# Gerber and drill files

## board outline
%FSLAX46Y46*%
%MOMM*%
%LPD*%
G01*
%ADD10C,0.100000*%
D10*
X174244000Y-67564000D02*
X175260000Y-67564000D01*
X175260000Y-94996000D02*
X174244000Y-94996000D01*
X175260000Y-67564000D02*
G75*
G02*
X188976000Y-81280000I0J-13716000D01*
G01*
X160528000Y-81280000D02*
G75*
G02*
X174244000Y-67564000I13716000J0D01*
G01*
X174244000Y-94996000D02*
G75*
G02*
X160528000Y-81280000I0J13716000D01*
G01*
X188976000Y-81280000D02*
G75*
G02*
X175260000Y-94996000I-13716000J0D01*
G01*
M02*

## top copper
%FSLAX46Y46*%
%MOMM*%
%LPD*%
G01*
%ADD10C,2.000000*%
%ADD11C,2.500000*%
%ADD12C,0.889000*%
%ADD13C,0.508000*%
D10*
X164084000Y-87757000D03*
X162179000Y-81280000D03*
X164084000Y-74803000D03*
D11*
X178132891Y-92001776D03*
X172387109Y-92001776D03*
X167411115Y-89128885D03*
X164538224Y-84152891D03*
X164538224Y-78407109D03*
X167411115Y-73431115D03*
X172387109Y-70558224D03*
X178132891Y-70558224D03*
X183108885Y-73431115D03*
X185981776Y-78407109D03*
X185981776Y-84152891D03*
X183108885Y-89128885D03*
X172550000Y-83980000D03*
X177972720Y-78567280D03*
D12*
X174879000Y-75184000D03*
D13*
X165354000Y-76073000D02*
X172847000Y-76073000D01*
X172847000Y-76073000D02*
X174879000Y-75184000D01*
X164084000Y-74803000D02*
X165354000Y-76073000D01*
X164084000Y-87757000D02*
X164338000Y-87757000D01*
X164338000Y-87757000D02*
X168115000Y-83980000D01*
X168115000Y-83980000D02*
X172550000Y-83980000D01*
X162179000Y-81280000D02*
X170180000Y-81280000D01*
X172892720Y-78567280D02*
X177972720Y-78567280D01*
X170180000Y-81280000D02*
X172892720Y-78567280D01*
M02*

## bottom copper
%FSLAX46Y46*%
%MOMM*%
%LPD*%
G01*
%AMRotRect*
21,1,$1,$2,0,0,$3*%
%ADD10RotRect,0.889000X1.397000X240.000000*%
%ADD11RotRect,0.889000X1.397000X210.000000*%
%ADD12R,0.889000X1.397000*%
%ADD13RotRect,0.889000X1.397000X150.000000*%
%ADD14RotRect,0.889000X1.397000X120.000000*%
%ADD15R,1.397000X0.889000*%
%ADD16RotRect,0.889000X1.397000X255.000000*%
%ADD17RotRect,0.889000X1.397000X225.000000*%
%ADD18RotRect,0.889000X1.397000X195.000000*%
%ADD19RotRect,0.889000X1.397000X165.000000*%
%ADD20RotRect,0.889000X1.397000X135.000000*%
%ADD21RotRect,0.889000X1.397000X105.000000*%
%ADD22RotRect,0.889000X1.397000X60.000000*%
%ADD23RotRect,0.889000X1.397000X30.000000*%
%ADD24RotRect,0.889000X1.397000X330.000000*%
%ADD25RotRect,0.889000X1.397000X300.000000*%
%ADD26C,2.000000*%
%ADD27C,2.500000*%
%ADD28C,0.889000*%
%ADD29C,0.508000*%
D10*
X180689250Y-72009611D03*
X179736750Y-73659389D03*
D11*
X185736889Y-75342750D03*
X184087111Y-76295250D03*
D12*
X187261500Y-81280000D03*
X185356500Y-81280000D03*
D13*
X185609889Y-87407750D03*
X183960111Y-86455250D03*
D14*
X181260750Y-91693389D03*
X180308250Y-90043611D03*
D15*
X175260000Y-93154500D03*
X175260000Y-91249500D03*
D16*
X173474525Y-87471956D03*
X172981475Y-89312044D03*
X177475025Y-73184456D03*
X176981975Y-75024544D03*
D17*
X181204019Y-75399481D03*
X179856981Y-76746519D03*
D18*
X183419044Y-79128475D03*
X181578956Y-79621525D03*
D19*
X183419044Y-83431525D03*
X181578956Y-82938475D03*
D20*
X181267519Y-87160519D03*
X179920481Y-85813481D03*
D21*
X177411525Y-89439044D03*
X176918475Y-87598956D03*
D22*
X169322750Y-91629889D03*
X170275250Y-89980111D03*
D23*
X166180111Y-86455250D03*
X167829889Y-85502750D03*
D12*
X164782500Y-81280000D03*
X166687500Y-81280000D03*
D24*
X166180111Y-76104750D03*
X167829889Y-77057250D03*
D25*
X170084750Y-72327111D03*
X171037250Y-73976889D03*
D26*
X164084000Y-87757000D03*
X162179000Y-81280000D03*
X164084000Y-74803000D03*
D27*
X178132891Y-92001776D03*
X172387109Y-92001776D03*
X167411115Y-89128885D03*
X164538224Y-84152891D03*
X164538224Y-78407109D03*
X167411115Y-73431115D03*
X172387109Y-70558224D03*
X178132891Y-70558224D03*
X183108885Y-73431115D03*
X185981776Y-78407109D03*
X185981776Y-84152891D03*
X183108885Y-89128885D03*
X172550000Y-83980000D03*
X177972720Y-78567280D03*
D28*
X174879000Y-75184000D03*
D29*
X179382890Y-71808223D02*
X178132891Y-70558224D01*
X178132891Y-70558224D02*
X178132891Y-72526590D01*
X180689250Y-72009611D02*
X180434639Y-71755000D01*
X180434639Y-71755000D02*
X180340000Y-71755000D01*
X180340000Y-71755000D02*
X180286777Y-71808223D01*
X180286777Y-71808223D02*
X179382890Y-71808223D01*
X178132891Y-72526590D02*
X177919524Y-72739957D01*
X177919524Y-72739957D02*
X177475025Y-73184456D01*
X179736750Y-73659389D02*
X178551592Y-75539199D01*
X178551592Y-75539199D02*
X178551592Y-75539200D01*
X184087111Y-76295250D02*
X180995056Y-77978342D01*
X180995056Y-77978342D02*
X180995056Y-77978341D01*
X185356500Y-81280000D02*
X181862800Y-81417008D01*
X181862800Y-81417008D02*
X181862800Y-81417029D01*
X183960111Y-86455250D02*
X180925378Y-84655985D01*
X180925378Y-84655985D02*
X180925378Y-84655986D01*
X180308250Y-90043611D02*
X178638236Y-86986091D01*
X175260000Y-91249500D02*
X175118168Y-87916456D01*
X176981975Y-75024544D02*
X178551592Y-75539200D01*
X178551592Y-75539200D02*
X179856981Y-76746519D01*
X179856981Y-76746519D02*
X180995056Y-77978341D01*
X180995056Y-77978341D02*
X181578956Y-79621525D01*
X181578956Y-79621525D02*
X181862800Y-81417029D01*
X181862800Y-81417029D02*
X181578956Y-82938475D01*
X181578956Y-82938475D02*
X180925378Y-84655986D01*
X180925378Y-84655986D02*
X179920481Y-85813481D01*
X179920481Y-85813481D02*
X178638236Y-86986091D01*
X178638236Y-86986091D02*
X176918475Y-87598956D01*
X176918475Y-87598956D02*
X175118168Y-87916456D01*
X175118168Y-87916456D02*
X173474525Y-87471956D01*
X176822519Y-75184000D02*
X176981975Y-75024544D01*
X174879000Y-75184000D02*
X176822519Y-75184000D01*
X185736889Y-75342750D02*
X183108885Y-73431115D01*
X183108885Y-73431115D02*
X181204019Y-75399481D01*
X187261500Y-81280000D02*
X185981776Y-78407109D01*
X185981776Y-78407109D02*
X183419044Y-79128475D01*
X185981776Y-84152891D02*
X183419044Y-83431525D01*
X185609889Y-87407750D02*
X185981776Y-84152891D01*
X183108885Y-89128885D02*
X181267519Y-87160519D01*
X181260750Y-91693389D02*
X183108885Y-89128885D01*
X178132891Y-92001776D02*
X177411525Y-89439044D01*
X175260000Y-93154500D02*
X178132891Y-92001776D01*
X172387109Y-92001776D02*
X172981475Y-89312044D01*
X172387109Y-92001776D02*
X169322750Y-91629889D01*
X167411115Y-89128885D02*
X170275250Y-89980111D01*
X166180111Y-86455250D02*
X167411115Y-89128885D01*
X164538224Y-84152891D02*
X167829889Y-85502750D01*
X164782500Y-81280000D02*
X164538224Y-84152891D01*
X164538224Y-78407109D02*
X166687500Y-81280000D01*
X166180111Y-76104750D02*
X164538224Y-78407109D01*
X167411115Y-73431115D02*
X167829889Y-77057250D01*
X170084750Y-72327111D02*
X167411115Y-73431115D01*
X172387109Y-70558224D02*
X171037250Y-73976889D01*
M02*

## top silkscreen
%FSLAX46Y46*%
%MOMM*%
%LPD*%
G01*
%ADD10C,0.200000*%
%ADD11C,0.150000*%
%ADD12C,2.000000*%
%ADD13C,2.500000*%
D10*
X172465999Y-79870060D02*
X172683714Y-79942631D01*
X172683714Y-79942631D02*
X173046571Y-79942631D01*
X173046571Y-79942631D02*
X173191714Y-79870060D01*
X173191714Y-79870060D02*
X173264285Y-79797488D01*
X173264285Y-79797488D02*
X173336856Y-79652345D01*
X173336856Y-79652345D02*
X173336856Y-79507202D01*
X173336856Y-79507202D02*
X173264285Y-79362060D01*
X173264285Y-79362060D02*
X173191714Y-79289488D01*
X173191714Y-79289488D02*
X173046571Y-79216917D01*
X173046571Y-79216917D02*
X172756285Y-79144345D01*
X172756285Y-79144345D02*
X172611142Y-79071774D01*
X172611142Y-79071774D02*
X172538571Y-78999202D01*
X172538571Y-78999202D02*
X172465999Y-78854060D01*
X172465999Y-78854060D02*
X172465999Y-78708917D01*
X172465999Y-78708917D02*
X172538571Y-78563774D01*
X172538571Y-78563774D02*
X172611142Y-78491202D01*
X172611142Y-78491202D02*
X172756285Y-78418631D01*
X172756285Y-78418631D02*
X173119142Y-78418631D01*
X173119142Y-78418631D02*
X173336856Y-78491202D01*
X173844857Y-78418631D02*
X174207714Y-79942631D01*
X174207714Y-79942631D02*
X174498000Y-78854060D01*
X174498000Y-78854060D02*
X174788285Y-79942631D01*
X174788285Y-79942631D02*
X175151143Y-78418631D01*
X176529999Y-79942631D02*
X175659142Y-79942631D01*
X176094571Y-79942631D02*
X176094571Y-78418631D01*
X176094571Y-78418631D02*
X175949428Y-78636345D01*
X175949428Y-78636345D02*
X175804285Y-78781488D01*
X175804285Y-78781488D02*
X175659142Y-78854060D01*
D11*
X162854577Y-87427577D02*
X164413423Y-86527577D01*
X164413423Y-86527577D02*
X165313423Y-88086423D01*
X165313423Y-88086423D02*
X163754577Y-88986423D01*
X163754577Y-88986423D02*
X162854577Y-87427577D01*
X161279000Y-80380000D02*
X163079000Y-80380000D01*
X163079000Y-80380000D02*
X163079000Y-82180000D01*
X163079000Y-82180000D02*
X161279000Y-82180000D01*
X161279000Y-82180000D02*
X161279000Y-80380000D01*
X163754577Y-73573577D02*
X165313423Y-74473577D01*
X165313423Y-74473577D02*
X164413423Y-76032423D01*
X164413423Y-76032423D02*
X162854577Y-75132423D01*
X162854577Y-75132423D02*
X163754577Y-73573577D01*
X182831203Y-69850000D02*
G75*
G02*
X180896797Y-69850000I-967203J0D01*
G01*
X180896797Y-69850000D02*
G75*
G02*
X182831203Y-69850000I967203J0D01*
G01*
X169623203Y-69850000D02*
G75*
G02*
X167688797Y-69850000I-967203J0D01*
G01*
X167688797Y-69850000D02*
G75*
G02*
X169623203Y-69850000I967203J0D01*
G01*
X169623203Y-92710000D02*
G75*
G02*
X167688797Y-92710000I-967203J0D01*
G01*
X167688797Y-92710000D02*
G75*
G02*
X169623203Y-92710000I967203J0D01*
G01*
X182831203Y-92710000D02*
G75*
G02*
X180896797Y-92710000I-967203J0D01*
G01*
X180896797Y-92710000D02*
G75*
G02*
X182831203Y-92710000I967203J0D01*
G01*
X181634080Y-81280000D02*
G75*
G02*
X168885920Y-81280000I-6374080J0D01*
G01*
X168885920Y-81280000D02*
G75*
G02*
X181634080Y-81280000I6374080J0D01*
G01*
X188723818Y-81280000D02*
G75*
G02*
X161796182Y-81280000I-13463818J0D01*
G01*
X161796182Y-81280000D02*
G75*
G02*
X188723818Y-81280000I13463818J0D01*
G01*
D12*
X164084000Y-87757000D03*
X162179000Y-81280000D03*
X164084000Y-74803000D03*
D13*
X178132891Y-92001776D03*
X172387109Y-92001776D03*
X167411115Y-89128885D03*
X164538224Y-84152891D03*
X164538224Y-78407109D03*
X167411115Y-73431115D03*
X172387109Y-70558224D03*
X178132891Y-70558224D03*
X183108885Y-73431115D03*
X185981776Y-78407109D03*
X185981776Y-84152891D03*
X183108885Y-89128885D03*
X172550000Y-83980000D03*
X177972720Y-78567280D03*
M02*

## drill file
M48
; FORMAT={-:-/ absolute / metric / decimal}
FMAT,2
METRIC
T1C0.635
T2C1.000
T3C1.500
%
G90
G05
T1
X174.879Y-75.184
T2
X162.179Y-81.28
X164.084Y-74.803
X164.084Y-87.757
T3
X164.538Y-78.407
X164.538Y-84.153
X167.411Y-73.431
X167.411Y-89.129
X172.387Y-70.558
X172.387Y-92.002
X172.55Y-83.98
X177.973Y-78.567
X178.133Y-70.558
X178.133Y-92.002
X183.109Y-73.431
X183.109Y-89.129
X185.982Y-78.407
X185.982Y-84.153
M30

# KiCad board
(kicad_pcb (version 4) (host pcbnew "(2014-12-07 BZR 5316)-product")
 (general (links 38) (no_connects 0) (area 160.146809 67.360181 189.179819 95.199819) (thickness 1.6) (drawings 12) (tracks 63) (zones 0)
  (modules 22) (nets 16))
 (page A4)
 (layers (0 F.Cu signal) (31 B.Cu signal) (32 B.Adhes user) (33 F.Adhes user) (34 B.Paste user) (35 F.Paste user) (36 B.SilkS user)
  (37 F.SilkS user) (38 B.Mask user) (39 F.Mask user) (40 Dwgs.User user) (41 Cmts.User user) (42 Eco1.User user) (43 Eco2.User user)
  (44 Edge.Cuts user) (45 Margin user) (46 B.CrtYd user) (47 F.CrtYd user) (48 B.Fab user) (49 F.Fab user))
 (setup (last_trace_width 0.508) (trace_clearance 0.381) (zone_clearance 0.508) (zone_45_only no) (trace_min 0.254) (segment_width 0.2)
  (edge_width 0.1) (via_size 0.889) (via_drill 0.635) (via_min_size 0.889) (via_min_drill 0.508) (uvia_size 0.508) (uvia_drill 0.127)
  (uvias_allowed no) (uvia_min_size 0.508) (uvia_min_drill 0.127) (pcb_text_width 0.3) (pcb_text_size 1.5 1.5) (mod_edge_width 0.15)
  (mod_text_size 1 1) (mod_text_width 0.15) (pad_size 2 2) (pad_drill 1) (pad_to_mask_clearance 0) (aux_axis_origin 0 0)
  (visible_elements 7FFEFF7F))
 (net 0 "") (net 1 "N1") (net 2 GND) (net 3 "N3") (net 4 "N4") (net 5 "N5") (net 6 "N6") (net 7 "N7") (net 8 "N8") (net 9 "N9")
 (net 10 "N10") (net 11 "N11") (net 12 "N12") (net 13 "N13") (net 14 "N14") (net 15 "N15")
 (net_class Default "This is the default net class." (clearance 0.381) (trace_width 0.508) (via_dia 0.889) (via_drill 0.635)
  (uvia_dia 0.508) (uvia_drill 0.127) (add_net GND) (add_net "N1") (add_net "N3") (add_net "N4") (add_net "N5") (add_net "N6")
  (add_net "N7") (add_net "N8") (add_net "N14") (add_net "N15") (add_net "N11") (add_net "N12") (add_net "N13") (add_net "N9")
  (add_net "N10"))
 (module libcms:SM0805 (layer B.Cu) (at 180.213 72.8345 240)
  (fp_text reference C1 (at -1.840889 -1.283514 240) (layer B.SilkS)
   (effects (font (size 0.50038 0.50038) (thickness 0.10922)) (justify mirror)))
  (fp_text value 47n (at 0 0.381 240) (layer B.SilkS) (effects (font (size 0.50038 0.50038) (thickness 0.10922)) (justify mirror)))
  (pad 1 smd rect (at -0.9525 0 240) (size 0.889 1.397) (layers B.Cu B.Paste B.Mask) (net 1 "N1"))
  (pad 2 smd rect (at 0.9525 0 240) (size 0.889 1.397) (layers B.Cu B.Paste B.Mask) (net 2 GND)))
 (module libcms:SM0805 (layer B.Cu) (at 184.912 75.819 210)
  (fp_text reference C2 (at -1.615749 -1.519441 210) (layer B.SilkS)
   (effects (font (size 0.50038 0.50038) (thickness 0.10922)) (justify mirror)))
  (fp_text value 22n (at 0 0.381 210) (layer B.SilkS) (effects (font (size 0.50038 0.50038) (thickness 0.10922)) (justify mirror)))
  (pad 1 smd rect (at -0.9525 0 210) (size 0.889 1.397) (layers B.Cu B.Paste B.Mask) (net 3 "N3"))
  (pad 2 smd rect (at 0.9525 0 210) (size 0.889 1.397) (layers B.Cu B.Paste B.Mask) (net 2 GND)))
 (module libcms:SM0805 (layer B.Cu) (at 186.309 81.28 180)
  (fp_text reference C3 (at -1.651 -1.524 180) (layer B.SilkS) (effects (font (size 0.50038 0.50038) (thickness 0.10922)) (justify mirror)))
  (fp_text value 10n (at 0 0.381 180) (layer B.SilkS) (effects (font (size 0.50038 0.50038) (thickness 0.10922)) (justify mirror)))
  (pad 1 smd rect (at -0.9525 0 180) (size 0.889 1.397) (layers B.Cu B.Paste B.Mask) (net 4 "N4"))
  (pad 2 smd rect (at 0.9525 0 180) (size 0.889 1.397) (layers B.Cu B.Paste B.Mask) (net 2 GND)))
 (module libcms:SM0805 (layer B.Cu) (at 184.785 86.9315 150)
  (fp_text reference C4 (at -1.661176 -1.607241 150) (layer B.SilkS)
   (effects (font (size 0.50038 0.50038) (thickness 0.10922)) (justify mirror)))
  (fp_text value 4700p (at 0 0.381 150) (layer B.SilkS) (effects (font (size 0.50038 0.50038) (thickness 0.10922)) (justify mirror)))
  (pad 1 smd rect (at -0.9525 0 150) (size 0.889 1.397) (layers B.Cu B.Paste B.Mask) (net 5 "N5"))
  (pad 2 smd rect (at 0.9525 0 150) (size 0.889 1.397) (layers B.Cu B.Paste B.Mask) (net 2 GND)))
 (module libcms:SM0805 (layer B.Cu) (at 180.7845 90.8685 120)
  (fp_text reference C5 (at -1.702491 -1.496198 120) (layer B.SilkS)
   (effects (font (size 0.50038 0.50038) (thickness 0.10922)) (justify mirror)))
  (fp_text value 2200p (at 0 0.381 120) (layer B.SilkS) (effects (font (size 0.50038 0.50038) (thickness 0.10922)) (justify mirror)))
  (pad 1 smd rect (at -0.9525 0 120) (size 0.889 1.397) (layers B.Cu B.Paste B.Mask) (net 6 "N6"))
  (pad 2 smd rect (at 0.9525 0 120) (size 0.889 1.397) (layers B.Cu B.Paste B.Mask) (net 2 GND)))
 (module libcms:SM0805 (layer B.Cu) (at 175.26 92.202 90)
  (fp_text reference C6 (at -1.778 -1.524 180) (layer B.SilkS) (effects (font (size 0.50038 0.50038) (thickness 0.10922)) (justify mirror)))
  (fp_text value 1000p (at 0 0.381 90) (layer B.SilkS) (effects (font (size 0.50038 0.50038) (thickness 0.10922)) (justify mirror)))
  (pad 1 smd rect (at -0.9525 0 90) (size 0.889 1.397) (layers B.Cu B.Paste B.Mask) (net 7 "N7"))
  (pad 2 smd rect (at 0.9525 0 90) (size 0.889 1.397) (layers B.Cu B.Paste B.Mask) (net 2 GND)))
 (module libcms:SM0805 (layer B.Cu) (at 173.228 88.392 255)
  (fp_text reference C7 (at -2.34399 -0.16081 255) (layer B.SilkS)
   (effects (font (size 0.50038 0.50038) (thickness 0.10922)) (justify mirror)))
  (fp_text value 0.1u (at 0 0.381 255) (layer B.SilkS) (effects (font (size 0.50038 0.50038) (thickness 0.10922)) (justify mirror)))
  (pad 1 smd rect (at -0.9525 0 255) (size 0.889 1.397) (layers B.Cu B.Paste B.Mask) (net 2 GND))
  (pad 2 smd rect (at 0.9525 0 255) (size 0.889 1.397) (layers B.Cu B.Paste B.Mask) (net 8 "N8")))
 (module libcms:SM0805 (layer B.Cu) (at 177.2285 74.1045 255)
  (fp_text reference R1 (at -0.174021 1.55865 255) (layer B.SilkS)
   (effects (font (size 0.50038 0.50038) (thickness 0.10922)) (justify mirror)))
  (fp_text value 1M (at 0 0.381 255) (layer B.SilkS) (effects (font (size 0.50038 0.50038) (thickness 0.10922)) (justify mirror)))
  (pad 1 smd rect (at -0.9525 0 255) (size 0.889 1.397) (layers B.Cu B.Paste B.Mask) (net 1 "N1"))
  (pad 2 smd rect (at 0.9525 0 255) (size 0.889 1.397) (layers B.Cu B.Paste B.Mask) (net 2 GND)))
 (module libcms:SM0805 (layer B.Cu) (at 180.5305 76.073 225)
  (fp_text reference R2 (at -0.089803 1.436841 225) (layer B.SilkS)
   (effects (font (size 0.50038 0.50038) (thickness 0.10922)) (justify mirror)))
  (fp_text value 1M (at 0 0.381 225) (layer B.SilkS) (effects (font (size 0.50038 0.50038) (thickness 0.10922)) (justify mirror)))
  (pad 1 smd rect (at -0.9525 0 225) (size 0.889 1.397) (layers B.Cu B.Paste B.Mask) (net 3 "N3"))
  (pad 2 smd rect (at 0.9525 0 225) (size 0.889 1.397) (layers B.Cu B.Paste B.Mask) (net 2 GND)))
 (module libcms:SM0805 (layer B.Cu) (at 182.499 79.375 195)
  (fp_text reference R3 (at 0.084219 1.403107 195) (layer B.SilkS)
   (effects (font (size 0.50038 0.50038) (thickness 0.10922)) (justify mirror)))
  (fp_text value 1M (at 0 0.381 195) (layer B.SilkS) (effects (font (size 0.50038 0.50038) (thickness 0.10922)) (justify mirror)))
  (pad 1 smd rect (at -0.9525 0 195) (size 0.889 1.397) (layers B.Cu B.Paste B.Mask) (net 4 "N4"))
  (pad 2 smd rect (at 0.9525 0 195) (size 0.889 1.397) (layers B.Cu B.Paste B.Mask) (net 2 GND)))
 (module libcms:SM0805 (layer B.Cu) (at 182.499 83.185 165)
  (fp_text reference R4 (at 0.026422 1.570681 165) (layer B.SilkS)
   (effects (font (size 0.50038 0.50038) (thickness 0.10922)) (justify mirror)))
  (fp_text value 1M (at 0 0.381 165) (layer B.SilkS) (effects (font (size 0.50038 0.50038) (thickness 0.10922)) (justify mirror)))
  (pad 1 smd rect (at -0.9525 0 165) (size 0.889 1.397) (layers B.Cu B.Paste B.Mask) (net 5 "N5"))
  (pad 2 smd rect (at 0.9525 0 165) (size 0.889 1.397) (layers B.Cu B.Paste B.Mask) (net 2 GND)))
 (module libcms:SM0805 (layer B.Cu) (at 180.594 86.487 135)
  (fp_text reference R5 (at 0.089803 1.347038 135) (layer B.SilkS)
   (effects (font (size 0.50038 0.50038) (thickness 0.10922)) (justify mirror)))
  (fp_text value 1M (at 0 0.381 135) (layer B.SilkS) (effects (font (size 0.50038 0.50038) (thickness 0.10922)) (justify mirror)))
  (pad 1 smd rect (at -0.9525 0 135) (size 0.889 1.397) (layers B.Cu B.Paste B.Mask) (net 6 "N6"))
  (pad 2 smd rect (at 0.9525 0 135) (size 0.889 1.397) (layers B.Cu B.Paste B.Mask) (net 2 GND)))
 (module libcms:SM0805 (layer B.Cu) (at 177.165 88.519 105)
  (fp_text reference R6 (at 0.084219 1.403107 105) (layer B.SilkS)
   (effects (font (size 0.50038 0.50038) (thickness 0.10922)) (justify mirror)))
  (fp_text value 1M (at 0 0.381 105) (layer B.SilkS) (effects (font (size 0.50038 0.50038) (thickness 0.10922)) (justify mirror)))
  (pad 1 smd rect (at -0.9525 0 105) (size 0.889 1.397) (layers B.Cu B.Paste B.Mask) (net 7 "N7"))
  (pad 2 smd rect (at 0.9525 0 105) (size 0.889 1.397) (layers B.Cu B.Paste B.Mask) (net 2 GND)))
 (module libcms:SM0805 (layer B.Cu) (at 169.799 90.805 60)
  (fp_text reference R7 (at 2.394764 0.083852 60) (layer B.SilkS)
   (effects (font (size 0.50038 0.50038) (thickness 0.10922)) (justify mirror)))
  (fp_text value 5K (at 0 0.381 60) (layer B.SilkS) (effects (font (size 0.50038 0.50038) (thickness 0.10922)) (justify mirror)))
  (pad 1 smd rect (at -0.9525 0 60) (size 0.889 1.397) (layers B.Cu B.Paste B.Mask) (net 8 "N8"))
  (pad 2 smd rect (at 0.9525 0 60) (size 0.889 1.397) (layers B.Cu B.Paste B.Mask) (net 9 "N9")))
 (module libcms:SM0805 (layer B.Cu) (at 167.005 85.979 30)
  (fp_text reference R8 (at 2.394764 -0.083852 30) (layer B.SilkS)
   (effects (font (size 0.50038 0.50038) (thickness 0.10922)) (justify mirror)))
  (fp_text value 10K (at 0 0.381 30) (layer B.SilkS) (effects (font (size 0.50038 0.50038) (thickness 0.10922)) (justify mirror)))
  (pad 1 smd rect (at -0.9525 0 30) (size 0.889 1.397) (layers B.Cu B.Paste B.Mask) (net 9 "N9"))
  (pad 2 smd rect (at 0.9525 0 30) (size 0.889 1.397) (layers B.Cu B.Paste B.Mask) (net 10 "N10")))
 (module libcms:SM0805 (layer B.Cu) (at 165.735 81.28)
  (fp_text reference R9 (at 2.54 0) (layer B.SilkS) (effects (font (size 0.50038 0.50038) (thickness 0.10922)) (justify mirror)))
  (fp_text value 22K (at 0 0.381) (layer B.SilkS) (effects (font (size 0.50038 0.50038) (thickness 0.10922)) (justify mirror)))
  (pad 1 smd rect (at -0.9525 0) (size 0.889 1.397) (layers B.Cu B.Paste B.Mask) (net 10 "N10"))
  (pad 2 smd rect (at 0.9525 0) (size 0.889 1.397) (layers B.Cu B.Paste B.Mask) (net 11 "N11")))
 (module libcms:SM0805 (layer B.Cu) (at 167.005 76.581 330)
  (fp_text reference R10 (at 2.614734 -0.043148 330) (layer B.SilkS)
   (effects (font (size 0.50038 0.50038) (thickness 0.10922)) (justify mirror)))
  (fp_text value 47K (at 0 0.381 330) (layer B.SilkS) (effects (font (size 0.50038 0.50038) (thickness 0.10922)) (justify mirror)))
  (pad 1 smd rect (at -0.9525 0 330) (size 0.889 1.397) (layers B.Cu B.Paste B.Mask) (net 11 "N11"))
  (pad 2 smd rect (at 0.9525 0 330) (size 0.889 1.397) (layers B.Cu B.Paste B.Mask) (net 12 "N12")))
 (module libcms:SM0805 (layer B.Cu) (at 170.561 73.152 300)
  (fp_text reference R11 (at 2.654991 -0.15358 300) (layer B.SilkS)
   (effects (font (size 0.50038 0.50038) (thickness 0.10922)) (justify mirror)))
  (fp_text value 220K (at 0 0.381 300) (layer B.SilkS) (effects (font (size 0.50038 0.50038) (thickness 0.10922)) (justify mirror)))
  (pad 1 smd rect (at -0.9525 0 300) (size 0.889 1.397) (layers B.Cu B.Paste B.Mask) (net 12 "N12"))
  (pad 2 smd rect (at 0.9525 0 300) (size 0.889 1.397) (layers B.Cu B.Paste B.Mask) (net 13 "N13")))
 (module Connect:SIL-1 (layer F.Cu) (at 164.084 87.757 30)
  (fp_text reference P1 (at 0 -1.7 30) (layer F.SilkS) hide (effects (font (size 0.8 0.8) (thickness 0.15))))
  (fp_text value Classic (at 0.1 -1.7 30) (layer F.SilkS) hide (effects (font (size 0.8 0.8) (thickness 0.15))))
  (fp_line (start -0.9 -0.9) (end 0.9 -0.9) (layer F.SilkS) (width 0.15))
  (fp_line (start 0.9 -0.9) (end 0.9 0.9) (layer F.SilkS) (width 0.15))
  (fp_line (start 0.9 0.9) (end -0.9 0.9) (layer F.SilkS) (width 0.15))
  (fp_line (start -0.9 0.9) (end -0.9 -0.9) (layer F.SilkS) (width 0.15))
  (pad 1 thru_hole circle (at 0 0 30) (size 2 2) (drill 1) (layers *.Cu *.Mask F.SilkS) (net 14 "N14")))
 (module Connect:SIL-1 (layer F.Cu) (at 162.179 81.28)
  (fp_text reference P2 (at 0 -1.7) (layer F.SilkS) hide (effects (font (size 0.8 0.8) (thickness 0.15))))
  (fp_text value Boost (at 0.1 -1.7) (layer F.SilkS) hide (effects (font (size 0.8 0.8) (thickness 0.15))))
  (fp_line (start -0.9 -0.9) (end 0.9 -0.9) (layer F.SilkS) (width 0.15))
  (fp_line (start 0.9 -0.9) (end 0.9 0.9) (layer F.SilkS) (width 0.15))
  (fp_line (start 0.9 0.9) (end -0.9 0.9) (layer F.SilkS) (width 0.15))
  (fp_line (start -0.9 0.9) (end -0.9 -0.9) (layer F.SilkS) (width 0.15))
  (pad 1 thru_hole circle (at 0 0) (size 2 2) (drill 1) (layers *.Cu *.Mask F.SilkS) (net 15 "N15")))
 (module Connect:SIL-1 (layer F.Cu) (at 164.084 74.803 330)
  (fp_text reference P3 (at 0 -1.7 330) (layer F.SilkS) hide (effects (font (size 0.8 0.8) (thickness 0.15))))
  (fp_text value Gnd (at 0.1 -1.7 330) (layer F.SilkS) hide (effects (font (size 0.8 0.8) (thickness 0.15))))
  (fp_line (start -0.9 -0.9) (end 0.9 -0.9) (layer F.SilkS) (width 0.15))
  (fp_line (start 0.9 -0.9) (end 0.9 0.9) (layer F.SilkS) (width 0.15))
  (fp_line (start 0.9 0.9) (end -0.9 0.9) (layer F.SilkS) (width 0.15))
  (fp_line (start -0.9 0.9) (end -0.9 -0.9) (layer F.SilkS) (width 0.15))
  (pad 1 thru_hole circle (at 0 0 330) (size 2 2) (drill 1) (layers *.Cu *.Mask F.SilkS) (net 2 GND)))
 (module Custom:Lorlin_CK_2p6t (layer F.Cu) (at 175.26 81.28)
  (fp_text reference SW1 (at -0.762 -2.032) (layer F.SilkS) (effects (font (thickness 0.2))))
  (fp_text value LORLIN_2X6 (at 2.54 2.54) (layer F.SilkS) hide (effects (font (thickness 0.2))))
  (fp_circle (center 6.604 -11.43) (end 7.493 -11.049) (layer F.SilkS) (width 0.15))
  (fp_circle (center -6.604 -11.43) (end -5.715 -11.049) (layer F.SilkS) (width 0.15))
  (fp_circle (center -6.604 11.43) (end -5.715 11.811) (layer F.SilkS) (width 0.15))
  (fp_circle (center 6.604 11.43) (end 7.493 11.811) (layer F.SilkS) (width 0.15))
  (fp_circle (center 0 0) (end 5.08 3.85) (layer F.SilkS) (width 0.15))
  (fp_circle (center 0 0) (end 11.1 7.62) (layer F.SilkS) (width 0.15))
  (pad 12 thru_hole circle (at 2.872891 10.721776) (size 2.5 2.5) (drill 1.5) (layers *.Cu *.Mask F.SilkS) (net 7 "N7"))
  (pad 1 thru_hole circle (at -2.872891 10.721776) (size 2.5 2.5) (drill 1.5) (layers *.Cu *.Mask F.SilkS) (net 8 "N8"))
  (pad 2 thru_hole circle (at -7.848885 7.848885) (size 2.5 2.5) (drill 1.5) (layers *.Cu *.Mask F.SilkS) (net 9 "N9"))
  (pad 3 thru_hole circle (at -10.721776 2.872891) (size 2.5 2.5) (drill 1.5) (layers *.Cu *.Mask F.SilkS) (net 10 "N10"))
  (pad 4 thru_hole circle (at -10.721776 -2.872891) (size 2.5 2.5) (drill 1.5) (layers *.Cu *.Mask F.SilkS) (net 11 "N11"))
  (pad 5 thru_hole circle (at -7.848885 -7.848885) (size 2.5 2.5) (drill 1.5) (layers *.Cu *.Mask F.SilkS) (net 12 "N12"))
  (pad 6 thru_hole circle (at -2.872891 -10.721776) (size 2.5 2.5) (drill 1.5) (layers *.Cu *.Mask F.SilkS) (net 13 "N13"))
  (pad 7 thru_hole circle (at 2.872891 -10.721776) (size 2.5 2.5) (drill 1.5) (layers *.Cu *.Mask F.SilkS) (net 1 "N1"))
  (pad 8 thru_hole circle (at 7.848885 -7.848885) (size 2.5 2.5) (drill 1.5) (layers *.Cu *.Mask F.SilkS) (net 3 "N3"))
  (pad 9 thru_hole circle (at 10.721776 -2.872891) (size 2.5 2.5) (drill 1.5) (layers *.Cu *.Mask F.SilkS) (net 4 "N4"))
  (pad 10 thru_hole circle (at 10.721776 2.872891) (size 2.5 2.5) (drill 1.5) (layers *.Cu *.Mask F.SilkS) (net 5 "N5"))
  (pad 11 thru_hole circle (at 7.848885 7.848885) (size 2.5 2.5) (drill 1.5) (layers *.Cu *.Mask F.SilkS) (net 6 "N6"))
  (pad A thru_hole circle (at -2.71 2.7) (size 2.5 2.5) (drill 1.5) (layers *.Cu *.Mask F.SilkS) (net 14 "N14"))
  (pad B thru_hole circle (at 2.71272 -2.71272) (size 2.5 2.5) (drill 1.5) (layers *.Cu *.Mask F.SilkS) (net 15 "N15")))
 (gr_line (start 174.244 67.564) (end 175.26 67.564) (angle 90) (layer Edge.Cuts) (width 0.1))
 (gr_line (start 175.26 94.996) (end 174.244 94.996) (angle 90) (layer Edge.Cuts) (width 0.1))
 (gr_arc (start 175.26 81.28) (end 175.26 67.564) (angle 90) (layer Edge.Cuts) (width 0.1))
 (gr_arc (start 174.244 81.28) (end 160.528 81.28) (angle 90) (layer Edge.Cuts) (width 0.1))
 (gr_arc (start 174.244 81.28) (end 174.244 94.996) (angle 90) (layer Edge.Cuts) (width 0.1))
 (gr_arc (start 175.26 81.28) (end 188.976 81.28) (angle 90) (layer Edge.Cuts) (width 0.1))
 (segment (start 179.38289 71.808223) (end 178.132891 70.558224) (width 0.508) (layer B.Cu) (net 1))
 (segment (start 178.132891 70.558224) (end 178.132891 72.52659) (width 0.508) (layer B.Cu) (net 1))
 (segment (start 180.68925 72.009611) (end 180.434639 71.755) (width 0.508) (layer B.Cu) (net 1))
 (segment (start 180.434639 71.755) (end 180.34 71.755) (width 0.508) (layer B.Cu) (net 1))
 (segment (start 180.34 71.755) (end 180.286777 71.808223) (width 0.508) (layer B.Cu) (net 1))
 (segment (start 180.286777 71.808223) (end 179.38289 71.808223) (width 0.508) (layer B.Cu) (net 1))
 (segment (start 178.132891 72.52659) (end 177.919524 72.739957) (width 0.508) (layer B.Cu) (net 1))
 (segment (start 177.919524 72.739957) (end 177.475025 73.184456) (width 0.508) (layer B.Cu) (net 1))
 (segment (start 179.73675 73.659389) (end 178.551592 75.539199) (width 0.508) (layer B.Cu) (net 2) (status 10))
 (segment (start 178.551592 75.539199) (end 178.551592 75.5392) (width 0.508) (layer B.Cu) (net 2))
 (segment (start 184.087111 76.29525) (end 180.995056 77.978342) (width 0.508) (layer B.Cu) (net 2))
 (segment (start 180.995056 77.978342) (end 180.995056 77.978341) (width 0.508) (layer B.Cu) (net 2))
 (segment (start 185.3565 81.28) (end 181.8628 81.417008) (width 0.508) (layer B.Cu) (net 2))
 (segment (start 181.8628 81.417008) (end 181.8628 81.417029) (width 0.508) (layer B.Cu) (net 2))
 (segment (start 183.960111 86.45525) (end 180.925378 84.655985) (width 0.508) (layer B.Cu) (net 2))
 (segment (start 180.925378 84.655985) (end 180.925378 84.655986) (width 0.508) (layer B.Cu) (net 2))
 (segment (start 180.30825 90.043611) (end 178.638236 86.986091) (width 0.508) (layer B.Cu) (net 2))
 (segment (start 175.26 91.2495) (end 175.118168 87.916456) (width 0.508) (layer B.Cu) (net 2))
 (segment (start 176.981975 75.024544) (end 178.551592 75.5392) (width 0.508) (layer B.Cu) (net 2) (status 10))
 (segment (start 178.551592 75.5392) (end 179.856981 76.746519) (width 0.508) (layer B.Cu) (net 2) (status 20))
 (segment (start 179.856981 76.746519) (end 180.995056 77.978341) (width 0.508) (layer B.Cu) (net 2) (status 10))
 (segment (start 180.995056 77.978341) (end 181.578956 79.621525) (width 0.508) (layer B.Cu) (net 2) (status 20))
 (segment (start 181.578956 79.621525) (end 181.8628 81.417029) (width 0.508) (layer B.Cu) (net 2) (status 10))
 (segment (start 181.8628 81.417029) (end 181.578956 82.938475) (width 0.508) (layer B.Cu) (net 2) (status 20))
 (segment (start 181.578956 82.938475) (end 180.925378 84.655986) (width 0.508) (layer B.Cu) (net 2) (status 10))
 (segment (start 180.925378 84.655986) (end 179.920481 85.813481) (width 0.508) (layer B.Cu) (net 2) (status 20))
 (segment (start 179.920481 85.813481) (end 178.638236 86.986091) (width 0.508) (layer B.Cu) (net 2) (status 10))
 (segment (start 178.638236 86.986091) (end 176.918475 87.598956) (width 0.508) (layer B.Cu) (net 2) (status 20))
 (segment (start 176.918475 87.598956) (end 175.118168 87.916456) (width 0.508) (layer B.Cu) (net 2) (status 10))
 (segment (start 175.118168 87.916456) (end 173.474525 87.471956) (width 0.508) (layer B.Cu) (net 2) (status 20))
 (segment (start 176.822519 75.184) (end 176.981975 75.024544) (width 0.508) (layer B.Cu) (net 2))
 (segment (start 165.354 76.073) (end 172.847 76.073) (width 0.508) (layer F.Cu) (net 2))
 (segment (start 172.847 76.073) (end 174.879 75.184) (width 0.508) (layer F.Cu) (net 2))
 (via (at 174.879 75.184) (size 0.889) (layers F.Cu B.Cu) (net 2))
 (segment (start 174.879 75.184) (end 176.822519 75.184) (width 0.508) (layer B.Cu) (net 2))
 (segment (start 164.084 74.803) (end 165.354 76.073) (width 0.508) (layer F.Cu) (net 2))
 (segment (start 185.736889 75.34275) (end 183.108885 73.431115) (width 0.508) (layer B.Cu) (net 3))
 (segment (start 183.108885 73.431115) (end 181.204019 75.399481) (width 0.508) (layer B.Cu) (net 3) (status 20))
 (segment (start 187.2615 81.28) (end 185.981776 78.407109) (width 0.508) (layer B.Cu) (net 4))
 (segment (start 185.981776 78.407109) (end 183.419044 79.128475) (width 0.508) (layer B.Cu) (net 4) (status 20))
 (segment (start 185.981776 84.152891) (end 183.419044 83.431525) (width 0.508) (layer B.Cu) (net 5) (status 20))
 (segment (start 185.609889 87.40775) (end 185.981776 84.152891) (width 0.508) (layer B.Cu) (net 5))
 (segment (start 183.108885 89.128885) (end 181.267519 87.160519) (width 0.508) (layer B.Cu) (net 6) (status 20))
 (segment (start 181.26075 91.693389) (end 183.108885 89.128885) (width 0.508) (layer B.Cu) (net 6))
 (segment (start 178.132891 92.001776) (end 177.411525 89.439044) (width 0.508) (layer B.Cu) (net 7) (status 20))
 (segment (start 175.26 93.1545) (end 178.132891 92.001776) (width 0.508) (layer B.Cu) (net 7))
 (segment (start 172.387109 92.001776) (end 172.981475 89.312044) (width 0.508) (layer B.Cu) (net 8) (status 20))
 (segment (start 172.387109 92.001776) (end 169.32275 91.629889) (width 0.508) (layer B.Cu) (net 8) (status 20))
 (segment (start 164.084 87.757) (end 164.338 87.757) (width 0.508) (layer F.Cu) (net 14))
 (segment (start 164.338 87.757) (end 168.115 83.98) (width 0.508) (layer F.Cu) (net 14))
 (segment (start 168.115 83.98) (end 172.55 83.98) (width 0.508) (layer F.Cu) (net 14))
 (segment (start 162.179 81.28) (end 170.18 81.28) (width 0.508) (layer F.Cu) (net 15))
 (segment (start 172.89272 78.56728) (end 177.97272 78.56728) (width 0.508) (layer F.Cu) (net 15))
 (segment (start 170.18 81.28) (end 172.89272 78.56728) (width 0.508) (layer F.Cu) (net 15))
 (segment (start 167.411115 89.128885) (end 170.27525 89.980111) (width 0.508) (layer B.Cu) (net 9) (status 20))
 (segment (start 166.180111 86.45525) (end 167.411115 89.128885) (width 0.508) (layer B.Cu) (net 9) (status 10))
 (segment (start 164.538224 84.152891) (end 167.829889 85.50275) (width 0.508) (layer B.Cu) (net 10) (status 20))
 (segment (start 164.7825 81.28) (end 164.538224 84.152891) (width 0.508) (layer B.Cu) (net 10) (status 10))
 (segment (start 164.538224 78.407109) (end 166.6875 81.28) (width 0.508) (layer B.Cu) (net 11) (status 20))
 (segment (start 166.180111 76.10475) (end 164.538224 78.407109) (width 0.508) (layer B.Cu) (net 11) (status 10))
 (segment (start 167.411115 73.431115) (end 167.829889 77.05725) (width 0.508) (layer B.Cu) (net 12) (status 20))
 (segment (start 170.08475 72.327111) (end 167.411115 73.431115) (width 0.508) (layer B.Cu) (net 12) (status 10))
 (segment (start 172.387109 70.558224) (end 171.03725 73.976889) (width 0.508) (layer B.Cu) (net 13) (status 20)))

